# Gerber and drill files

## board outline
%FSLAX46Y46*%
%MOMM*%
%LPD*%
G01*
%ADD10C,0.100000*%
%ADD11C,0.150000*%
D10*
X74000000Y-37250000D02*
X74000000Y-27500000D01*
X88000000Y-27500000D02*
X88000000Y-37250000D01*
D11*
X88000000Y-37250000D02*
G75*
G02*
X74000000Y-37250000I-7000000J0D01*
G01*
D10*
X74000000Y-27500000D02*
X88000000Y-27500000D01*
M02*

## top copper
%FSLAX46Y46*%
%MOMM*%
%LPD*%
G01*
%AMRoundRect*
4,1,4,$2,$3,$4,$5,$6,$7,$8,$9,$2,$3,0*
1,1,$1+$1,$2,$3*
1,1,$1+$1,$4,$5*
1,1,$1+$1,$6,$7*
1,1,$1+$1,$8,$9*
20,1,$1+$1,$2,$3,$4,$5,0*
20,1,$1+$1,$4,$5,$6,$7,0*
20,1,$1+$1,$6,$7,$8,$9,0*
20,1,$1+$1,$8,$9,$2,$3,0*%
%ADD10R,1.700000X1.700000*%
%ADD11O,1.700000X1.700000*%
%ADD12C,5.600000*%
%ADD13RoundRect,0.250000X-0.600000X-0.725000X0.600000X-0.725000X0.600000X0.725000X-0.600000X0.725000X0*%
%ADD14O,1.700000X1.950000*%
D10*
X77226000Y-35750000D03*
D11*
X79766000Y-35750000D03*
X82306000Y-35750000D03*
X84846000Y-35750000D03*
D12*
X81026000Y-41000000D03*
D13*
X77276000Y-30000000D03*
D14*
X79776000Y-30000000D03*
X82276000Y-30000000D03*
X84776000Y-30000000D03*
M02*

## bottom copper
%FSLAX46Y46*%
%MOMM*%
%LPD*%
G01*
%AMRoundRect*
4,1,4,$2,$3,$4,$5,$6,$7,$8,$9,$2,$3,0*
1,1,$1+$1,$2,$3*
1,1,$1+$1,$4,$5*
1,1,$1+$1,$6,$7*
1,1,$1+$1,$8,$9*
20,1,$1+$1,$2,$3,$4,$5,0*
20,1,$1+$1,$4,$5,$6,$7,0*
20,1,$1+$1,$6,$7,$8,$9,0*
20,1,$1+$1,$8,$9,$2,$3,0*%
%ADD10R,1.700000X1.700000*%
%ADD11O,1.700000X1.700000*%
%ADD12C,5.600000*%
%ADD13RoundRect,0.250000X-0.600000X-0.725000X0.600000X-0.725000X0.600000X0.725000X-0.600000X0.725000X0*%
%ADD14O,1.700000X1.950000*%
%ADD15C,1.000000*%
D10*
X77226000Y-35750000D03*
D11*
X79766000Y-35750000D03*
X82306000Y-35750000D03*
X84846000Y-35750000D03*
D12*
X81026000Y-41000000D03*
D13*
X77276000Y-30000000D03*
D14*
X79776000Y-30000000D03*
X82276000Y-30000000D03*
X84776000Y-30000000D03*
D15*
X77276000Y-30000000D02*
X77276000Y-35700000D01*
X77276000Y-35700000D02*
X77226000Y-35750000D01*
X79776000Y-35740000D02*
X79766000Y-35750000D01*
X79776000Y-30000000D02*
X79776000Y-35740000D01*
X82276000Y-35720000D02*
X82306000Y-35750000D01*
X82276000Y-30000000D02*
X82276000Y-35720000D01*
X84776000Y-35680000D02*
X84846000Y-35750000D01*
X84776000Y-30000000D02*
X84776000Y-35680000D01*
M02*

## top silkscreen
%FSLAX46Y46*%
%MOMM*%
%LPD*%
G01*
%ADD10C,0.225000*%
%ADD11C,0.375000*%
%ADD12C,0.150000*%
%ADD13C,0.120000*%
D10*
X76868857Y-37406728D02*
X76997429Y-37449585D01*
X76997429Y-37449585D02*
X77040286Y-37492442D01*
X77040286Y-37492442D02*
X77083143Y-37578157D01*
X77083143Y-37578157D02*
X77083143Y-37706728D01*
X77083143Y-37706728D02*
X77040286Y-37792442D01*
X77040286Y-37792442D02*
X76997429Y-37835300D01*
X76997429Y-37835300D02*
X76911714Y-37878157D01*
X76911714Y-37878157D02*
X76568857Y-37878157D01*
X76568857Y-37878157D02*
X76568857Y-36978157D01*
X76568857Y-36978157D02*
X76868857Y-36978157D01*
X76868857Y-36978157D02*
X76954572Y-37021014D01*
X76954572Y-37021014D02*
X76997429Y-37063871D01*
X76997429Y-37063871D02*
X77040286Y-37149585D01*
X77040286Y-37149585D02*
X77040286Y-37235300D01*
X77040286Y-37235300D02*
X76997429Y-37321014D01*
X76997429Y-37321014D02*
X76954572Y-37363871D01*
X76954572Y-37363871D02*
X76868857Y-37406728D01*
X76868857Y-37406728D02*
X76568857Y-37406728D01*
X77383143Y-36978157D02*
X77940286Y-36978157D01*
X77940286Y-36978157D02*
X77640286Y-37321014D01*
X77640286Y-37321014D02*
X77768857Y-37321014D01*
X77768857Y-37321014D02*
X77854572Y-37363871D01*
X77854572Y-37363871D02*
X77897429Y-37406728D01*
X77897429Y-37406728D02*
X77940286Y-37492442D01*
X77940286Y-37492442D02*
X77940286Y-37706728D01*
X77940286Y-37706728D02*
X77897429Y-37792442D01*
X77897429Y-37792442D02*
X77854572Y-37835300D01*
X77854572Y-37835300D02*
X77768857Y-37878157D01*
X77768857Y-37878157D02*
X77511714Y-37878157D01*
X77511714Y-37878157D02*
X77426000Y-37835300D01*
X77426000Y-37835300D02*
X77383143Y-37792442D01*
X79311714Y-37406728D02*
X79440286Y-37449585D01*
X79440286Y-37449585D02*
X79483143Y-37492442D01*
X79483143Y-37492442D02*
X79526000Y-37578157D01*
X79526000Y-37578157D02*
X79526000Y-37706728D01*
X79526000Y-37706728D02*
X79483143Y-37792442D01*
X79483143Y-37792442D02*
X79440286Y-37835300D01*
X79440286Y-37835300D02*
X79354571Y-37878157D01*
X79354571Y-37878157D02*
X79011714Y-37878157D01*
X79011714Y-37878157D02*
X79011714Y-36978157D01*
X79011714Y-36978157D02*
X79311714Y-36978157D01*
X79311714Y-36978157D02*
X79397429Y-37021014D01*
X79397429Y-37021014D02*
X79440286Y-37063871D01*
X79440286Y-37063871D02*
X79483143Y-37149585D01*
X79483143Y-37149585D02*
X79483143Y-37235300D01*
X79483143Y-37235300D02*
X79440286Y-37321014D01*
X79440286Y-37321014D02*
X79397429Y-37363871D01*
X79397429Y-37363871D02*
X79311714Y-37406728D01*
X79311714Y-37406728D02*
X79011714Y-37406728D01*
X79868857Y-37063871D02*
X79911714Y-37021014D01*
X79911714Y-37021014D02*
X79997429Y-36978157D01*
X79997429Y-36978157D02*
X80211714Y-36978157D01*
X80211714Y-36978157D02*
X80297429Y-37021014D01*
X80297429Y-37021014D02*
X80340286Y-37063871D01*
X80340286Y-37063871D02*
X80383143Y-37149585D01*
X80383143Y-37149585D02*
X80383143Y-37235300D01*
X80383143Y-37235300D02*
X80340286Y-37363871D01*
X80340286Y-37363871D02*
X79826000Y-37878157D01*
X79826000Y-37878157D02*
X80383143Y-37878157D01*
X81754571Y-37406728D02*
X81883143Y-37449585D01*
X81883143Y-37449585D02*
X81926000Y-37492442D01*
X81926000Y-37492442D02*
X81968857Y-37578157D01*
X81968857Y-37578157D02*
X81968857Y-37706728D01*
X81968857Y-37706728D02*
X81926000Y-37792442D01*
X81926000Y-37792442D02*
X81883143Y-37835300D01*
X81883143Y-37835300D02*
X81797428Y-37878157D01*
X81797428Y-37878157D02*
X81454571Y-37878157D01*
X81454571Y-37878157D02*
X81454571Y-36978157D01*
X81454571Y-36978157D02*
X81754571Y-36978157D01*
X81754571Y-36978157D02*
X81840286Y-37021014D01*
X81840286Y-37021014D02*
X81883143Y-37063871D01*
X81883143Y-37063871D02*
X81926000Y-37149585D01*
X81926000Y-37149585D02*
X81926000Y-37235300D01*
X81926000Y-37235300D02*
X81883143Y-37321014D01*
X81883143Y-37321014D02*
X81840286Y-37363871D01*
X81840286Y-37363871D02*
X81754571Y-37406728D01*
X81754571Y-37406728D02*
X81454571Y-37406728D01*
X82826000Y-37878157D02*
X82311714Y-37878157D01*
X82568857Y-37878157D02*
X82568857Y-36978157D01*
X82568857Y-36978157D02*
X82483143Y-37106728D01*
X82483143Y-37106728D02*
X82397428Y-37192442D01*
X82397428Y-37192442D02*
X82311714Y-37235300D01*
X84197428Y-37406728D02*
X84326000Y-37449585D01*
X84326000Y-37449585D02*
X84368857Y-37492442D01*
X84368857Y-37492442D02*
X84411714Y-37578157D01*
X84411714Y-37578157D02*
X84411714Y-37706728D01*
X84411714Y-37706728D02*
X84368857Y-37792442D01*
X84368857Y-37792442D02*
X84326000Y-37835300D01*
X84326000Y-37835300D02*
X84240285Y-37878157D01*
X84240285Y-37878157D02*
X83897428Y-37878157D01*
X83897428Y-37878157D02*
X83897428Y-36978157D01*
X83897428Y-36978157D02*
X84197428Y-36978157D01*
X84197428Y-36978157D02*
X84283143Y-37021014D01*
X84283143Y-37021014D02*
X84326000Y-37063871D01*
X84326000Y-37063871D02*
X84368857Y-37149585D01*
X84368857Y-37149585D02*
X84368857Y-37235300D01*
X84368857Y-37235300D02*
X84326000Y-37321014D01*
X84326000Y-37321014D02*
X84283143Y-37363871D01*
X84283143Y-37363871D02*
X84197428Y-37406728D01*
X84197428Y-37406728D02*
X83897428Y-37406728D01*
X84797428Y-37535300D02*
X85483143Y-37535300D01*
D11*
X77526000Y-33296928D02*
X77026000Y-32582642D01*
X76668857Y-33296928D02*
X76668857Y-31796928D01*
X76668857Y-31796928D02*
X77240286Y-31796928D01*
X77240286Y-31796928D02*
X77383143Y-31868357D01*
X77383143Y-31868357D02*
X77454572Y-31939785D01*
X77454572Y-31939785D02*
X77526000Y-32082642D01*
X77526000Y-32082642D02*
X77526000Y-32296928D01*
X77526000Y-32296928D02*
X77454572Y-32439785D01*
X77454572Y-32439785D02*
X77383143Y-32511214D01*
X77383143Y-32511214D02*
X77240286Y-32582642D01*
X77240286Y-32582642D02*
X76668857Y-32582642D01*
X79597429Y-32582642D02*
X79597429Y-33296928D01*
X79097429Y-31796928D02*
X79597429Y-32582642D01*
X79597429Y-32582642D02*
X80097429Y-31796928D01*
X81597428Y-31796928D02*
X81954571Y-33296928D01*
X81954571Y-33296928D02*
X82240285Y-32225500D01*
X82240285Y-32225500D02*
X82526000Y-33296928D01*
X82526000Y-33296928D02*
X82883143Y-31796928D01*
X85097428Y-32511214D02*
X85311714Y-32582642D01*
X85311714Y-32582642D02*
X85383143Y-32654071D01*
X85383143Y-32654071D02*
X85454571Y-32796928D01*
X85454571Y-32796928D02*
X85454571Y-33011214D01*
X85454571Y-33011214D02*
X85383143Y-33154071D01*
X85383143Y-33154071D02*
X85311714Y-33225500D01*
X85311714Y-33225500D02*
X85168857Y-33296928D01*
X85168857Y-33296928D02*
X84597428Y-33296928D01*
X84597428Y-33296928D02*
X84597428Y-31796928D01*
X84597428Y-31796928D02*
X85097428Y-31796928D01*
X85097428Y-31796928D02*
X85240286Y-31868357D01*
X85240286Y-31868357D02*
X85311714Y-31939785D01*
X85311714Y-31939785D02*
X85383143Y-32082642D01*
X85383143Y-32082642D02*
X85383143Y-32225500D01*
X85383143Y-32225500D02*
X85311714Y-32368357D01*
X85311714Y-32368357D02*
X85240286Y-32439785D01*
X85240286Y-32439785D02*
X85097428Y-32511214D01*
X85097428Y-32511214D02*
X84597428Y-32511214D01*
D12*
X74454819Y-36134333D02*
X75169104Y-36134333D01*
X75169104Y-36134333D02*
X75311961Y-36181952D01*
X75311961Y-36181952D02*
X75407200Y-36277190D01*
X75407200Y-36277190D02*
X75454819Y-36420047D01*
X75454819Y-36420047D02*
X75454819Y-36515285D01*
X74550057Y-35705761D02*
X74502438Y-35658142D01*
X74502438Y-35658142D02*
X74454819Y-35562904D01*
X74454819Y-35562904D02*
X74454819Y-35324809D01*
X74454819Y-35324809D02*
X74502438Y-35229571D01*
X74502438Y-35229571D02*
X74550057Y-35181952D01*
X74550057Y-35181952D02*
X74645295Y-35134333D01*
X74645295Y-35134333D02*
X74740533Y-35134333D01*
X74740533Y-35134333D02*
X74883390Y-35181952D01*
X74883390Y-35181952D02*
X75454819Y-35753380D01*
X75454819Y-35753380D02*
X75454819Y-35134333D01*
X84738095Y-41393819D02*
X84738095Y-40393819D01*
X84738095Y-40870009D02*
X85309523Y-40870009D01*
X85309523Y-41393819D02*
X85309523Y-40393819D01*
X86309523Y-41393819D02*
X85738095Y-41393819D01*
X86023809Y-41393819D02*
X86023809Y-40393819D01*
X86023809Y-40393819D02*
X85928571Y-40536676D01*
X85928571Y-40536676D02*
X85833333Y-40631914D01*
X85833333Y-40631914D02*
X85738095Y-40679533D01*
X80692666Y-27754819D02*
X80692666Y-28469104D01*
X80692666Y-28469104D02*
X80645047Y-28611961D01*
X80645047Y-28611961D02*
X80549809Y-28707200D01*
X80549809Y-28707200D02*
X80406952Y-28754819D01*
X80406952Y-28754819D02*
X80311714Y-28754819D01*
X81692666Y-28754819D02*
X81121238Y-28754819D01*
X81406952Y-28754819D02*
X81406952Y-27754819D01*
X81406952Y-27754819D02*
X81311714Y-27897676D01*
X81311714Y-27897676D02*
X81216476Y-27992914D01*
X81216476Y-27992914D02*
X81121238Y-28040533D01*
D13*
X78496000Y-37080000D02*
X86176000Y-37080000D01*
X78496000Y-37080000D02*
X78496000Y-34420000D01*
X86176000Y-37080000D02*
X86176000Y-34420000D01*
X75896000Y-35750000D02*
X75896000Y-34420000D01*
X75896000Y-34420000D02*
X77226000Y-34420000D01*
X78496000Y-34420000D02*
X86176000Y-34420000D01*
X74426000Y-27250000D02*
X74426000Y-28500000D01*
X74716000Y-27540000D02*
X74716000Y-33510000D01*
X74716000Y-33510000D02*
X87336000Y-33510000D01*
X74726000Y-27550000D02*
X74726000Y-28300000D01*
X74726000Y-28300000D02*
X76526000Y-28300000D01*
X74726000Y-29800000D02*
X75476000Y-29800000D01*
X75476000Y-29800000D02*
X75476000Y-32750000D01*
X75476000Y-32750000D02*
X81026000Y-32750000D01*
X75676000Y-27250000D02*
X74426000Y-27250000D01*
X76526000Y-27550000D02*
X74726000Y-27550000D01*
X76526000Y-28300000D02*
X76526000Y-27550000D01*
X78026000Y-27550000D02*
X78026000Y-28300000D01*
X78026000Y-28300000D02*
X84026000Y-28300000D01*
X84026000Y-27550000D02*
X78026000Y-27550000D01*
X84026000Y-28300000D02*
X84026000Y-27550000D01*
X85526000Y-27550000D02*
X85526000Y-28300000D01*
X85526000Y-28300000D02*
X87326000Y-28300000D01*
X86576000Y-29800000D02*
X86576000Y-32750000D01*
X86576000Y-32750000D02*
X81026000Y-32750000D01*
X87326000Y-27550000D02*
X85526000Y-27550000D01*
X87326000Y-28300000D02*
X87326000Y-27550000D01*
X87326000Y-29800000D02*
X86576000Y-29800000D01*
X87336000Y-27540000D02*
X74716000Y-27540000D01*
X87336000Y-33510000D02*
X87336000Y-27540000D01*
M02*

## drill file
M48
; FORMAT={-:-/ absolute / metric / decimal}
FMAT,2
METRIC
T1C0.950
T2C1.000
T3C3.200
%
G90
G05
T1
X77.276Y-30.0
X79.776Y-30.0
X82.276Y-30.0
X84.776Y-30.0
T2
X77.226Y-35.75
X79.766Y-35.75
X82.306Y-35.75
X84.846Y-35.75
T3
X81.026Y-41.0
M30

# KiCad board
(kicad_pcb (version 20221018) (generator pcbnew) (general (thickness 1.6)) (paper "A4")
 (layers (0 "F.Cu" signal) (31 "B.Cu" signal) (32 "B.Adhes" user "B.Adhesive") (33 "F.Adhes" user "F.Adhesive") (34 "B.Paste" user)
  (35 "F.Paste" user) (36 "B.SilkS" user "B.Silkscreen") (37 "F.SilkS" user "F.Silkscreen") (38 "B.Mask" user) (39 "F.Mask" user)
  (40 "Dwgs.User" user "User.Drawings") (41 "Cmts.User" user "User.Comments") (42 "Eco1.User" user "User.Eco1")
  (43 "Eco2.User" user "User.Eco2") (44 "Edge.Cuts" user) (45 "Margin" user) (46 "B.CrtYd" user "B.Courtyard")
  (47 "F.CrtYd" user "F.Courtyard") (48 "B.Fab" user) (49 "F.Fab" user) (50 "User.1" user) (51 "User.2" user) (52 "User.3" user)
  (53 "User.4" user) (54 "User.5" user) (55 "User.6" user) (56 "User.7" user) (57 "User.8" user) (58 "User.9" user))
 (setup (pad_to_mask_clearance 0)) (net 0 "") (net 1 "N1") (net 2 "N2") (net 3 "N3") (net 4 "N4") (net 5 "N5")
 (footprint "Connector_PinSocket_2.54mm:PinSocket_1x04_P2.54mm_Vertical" (layer "F.Cu") (at 77.226 35.75 90)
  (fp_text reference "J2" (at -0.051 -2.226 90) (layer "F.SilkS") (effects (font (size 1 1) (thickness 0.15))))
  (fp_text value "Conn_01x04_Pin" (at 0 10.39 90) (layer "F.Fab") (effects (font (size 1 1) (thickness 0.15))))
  (fp_line (start -1.33 1.27) (end -1.33 8.95) (stroke (width 0.12) (type solid)) (layer "F.SilkS"))
  (fp_line (start -1.33 1.27) (end 1.33 1.27) (stroke (width 0.12) (type solid)) (layer "F.SilkS"))
  (fp_line (start -1.33 8.95) (end 1.33 8.95) (stroke (width 0.12) (type solid)) (layer "F.SilkS"))
  (fp_line (start 0 -1.33) (end 1.33 -1.33) (stroke (width 0.12) (type solid)) (layer "F.SilkS"))
  (fp_line (start 1.33 -1.33) (end 1.33 0) (stroke (width 0.12) (type solid)) (layer "F.SilkS"))
  (fp_line (start 1.33 1.27) (end 1.33 8.95) (stroke (width 0.12) (type solid)) (layer "F.SilkS"))
  (pad "1" thru_hole rect (at 0 0 90) (size 1.7 1.7) (drill 1) (layers "*.Cu" "*.Mask") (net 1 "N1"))
  (pad "2" thru_hole oval (at 0 2.54 90) (size 1.7 1.7) (drill 1) (layers "*.Cu" "*.Mask") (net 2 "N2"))
  (pad "3" thru_hole oval (at 0 5.08 90) (size 1.7 1.7) (drill 1) (layers "*.Cu" "*.Mask") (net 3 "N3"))
  (pad "4" thru_hole oval (at 0 7.62 90) (size 1.7 1.7) (drill 1) (layers "*.Cu" "*.Mask") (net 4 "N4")))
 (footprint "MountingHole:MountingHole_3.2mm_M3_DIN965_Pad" (layer "F.Cu") (at 81.026 41)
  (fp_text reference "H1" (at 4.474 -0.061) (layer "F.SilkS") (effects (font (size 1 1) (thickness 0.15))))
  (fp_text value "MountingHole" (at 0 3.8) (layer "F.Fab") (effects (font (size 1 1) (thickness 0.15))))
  (pad "1" thru_hole circle (at 0 0) (size 5.6 5.6) (drill 3.2) (layers "*.Cu" "*.Mask") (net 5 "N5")))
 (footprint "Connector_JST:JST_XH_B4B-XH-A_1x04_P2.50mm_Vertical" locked (layer "F.Cu") (at 77.276 30)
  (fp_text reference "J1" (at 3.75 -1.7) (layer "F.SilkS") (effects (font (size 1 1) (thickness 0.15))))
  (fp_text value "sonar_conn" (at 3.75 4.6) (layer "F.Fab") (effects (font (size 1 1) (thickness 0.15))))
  (fp_line (start -2.85 -2.75) (end -2.85 -1.5) (stroke (width 0.12) (type solid)) (layer "F.SilkS"))
  (fp_line (start -2.56 -2.46) (end -2.56 3.51) (stroke (width 0.12) (type solid)) (layer "F.SilkS"))
  (fp_line (start -2.56 3.51) (end 10.06 3.51) (stroke (width 0.12) (type solid)) (layer "F.SilkS"))
  (fp_line (start -2.55 -2.45) (end -2.55 -1.7) (stroke (width 0.12) (type solid)) (layer "F.SilkS"))
  (fp_line (start -2.55 -1.7) (end -0.75 -1.7) (stroke (width 0.12) (type solid)) (layer "F.SilkS"))
  (fp_line (start -2.55 -0.2) (end -1.8 -0.2) (stroke (width 0.12) (type solid)) (layer "F.SilkS"))
  (fp_line (start -1.8 -0.2) (end -1.8 2.75) (stroke (width 0.12) (type solid)) (layer "F.SilkS"))
  (fp_line (start -1.8 2.75) (end 3.75 2.75) (stroke (width 0.12) (type solid)) (layer "F.SilkS"))
  (fp_line (start -1.6 -2.75) (end -2.85 -2.75) (stroke (width 0.12) (type solid)) (layer "F.SilkS"))
  (fp_line (start -0.75 -2.45) (end -2.55 -2.45) (stroke (width 0.12) (type solid)) (layer "F.SilkS"))
  (fp_line (start -0.75 -1.7) (end -0.75 -2.45) (stroke (width 0.12) (type solid)) (layer "F.SilkS"))
  (fp_line (start 0.75 -2.45) (end 0.75 -1.7) (stroke (width 0.12) (type solid)) (layer "F.SilkS"))
  (fp_line (start 0.75 -1.7) (end 6.75 -1.7) (stroke (width 0.12) (type solid)) (layer "F.SilkS"))
  (fp_line (start 6.75 -2.45) (end 0.75 -2.45) (stroke (width 0.12) (type solid)) (layer "F.SilkS"))
  (fp_line (start 6.75 -1.7) (end 6.75 -2.45) (stroke (width 0.12) (type solid)) (layer "F.SilkS"))
  (fp_line (start 8.25 -2.45) (end 8.25 -1.7) (stroke (width 0.12) (type solid)) (layer "F.SilkS"))
  (fp_line (start 8.25 -1.7) (end 10.05 -1.7) (stroke (width 0.12) (type solid)) (layer "F.SilkS"))
  (fp_line (start 9.3 -0.2) (end 9.3 2.75) (stroke (width 0.12) (type solid)) (layer "F.SilkS"))
  (fp_line (start 9.3 2.75) (end 3.75 2.75) (stroke (width 0.12) (type solid)) (layer "F.SilkS"))
  (fp_line (start 10.05 -2.45) (end 8.25 -2.45) (stroke (width 0.12) (type solid)) (layer "F.SilkS"))
  (fp_line (start 10.05 -1.7) (end 10.05 -2.45) (stroke (width 0.12) (type solid)) (layer "F.SilkS"))
  (fp_line (start 10.05 -0.2) (end 9.3 -0.2) (stroke (width 0.12) (type solid)) (layer "F.SilkS"))
  (fp_line (start 10.06 -2.46) (end -2.56 -2.46) (stroke (width 0.12) (type solid)) (layer "F.SilkS"))
  (fp_line (start 10.06 3.51) (end 10.06 -2.46) (stroke (width 0.12) (type solid)) (layer "F.SilkS"))
  (pad "1" thru_hole roundrect locked (at 0 0) (size 1.7 1.95) (drill 0.95) (layers "*.Cu" "*.Mask") (roundrect_rratio 0.1470588235)
   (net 1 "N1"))
  (pad "2" thru_hole oval locked (at 2.5 0) (size 1.7 1.95) (drill 0.95) (layers "*.Cu" "*.Mask") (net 2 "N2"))
  (pad "3" thru_hole oval locked (at 5 0) (size 1.7 1.95) (drill 0.95) (layers "*.Cu" "*.Mask") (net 3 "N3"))
  (pad "4" thru_hole oval locked (at 7.5 0) (size 1.7 1.95) (drill 0.95) (layers "*.Cu" "*.Mask") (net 4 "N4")))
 (gr_line (start 74 37.25) (end 74 27.5) (stroke (width 0.1) (type default)) (layer "Edge.Cuts"))
 (gr_line (start 88 27.5) (end 88 37.25) (stroke (width 0.1) (type default)) (layer "Edge.Cuts"))
 (gr_arc (start 88 37.25) (mid 81 44.25) (end 74 37.25) (stroke (width 0.15) (type default)) (layer "Edge.Cuts"))
 (gr_line (start 74 27.5) (end 88 27.5) (stroke (width 0.1) (type default)) (layer "Edge.Cuts"))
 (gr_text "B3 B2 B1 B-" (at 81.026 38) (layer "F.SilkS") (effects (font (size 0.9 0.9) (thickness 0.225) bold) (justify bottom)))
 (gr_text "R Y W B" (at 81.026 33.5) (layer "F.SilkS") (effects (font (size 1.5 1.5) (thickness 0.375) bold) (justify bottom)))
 (segment (start 77.276 30) (end 77.276 35.7) (width 1) (layer "B.Cu") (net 1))
 (segment (start 77.276 35.7) (end 77.226 35.75) (width 1) (layer "B.Cu") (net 1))
 (segment (start 79.776 35.74) (end 79.766 35.75) (width 1) (layer "B.Cu") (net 2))
 (segment (start 79.776 30) (end 79.776 35.74) (width 1) (layer "B.Cu") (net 2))
 (segment (start 82.276 35.72) (end 82.306 35.75) (width 1) (layer "B.Cu") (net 3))
 (segment (start 82.276 30) (end 82.276 35.72) (width 1) (layer "B.Cu") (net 3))
 (segment (start 84.776 35.68) (end 84.846 35.75) (width 1) (layer "B.Cu") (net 4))
 (segment (start 84.776 30) (end 84.776 35.68) (width 1) (layer "B.Cu") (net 4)))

